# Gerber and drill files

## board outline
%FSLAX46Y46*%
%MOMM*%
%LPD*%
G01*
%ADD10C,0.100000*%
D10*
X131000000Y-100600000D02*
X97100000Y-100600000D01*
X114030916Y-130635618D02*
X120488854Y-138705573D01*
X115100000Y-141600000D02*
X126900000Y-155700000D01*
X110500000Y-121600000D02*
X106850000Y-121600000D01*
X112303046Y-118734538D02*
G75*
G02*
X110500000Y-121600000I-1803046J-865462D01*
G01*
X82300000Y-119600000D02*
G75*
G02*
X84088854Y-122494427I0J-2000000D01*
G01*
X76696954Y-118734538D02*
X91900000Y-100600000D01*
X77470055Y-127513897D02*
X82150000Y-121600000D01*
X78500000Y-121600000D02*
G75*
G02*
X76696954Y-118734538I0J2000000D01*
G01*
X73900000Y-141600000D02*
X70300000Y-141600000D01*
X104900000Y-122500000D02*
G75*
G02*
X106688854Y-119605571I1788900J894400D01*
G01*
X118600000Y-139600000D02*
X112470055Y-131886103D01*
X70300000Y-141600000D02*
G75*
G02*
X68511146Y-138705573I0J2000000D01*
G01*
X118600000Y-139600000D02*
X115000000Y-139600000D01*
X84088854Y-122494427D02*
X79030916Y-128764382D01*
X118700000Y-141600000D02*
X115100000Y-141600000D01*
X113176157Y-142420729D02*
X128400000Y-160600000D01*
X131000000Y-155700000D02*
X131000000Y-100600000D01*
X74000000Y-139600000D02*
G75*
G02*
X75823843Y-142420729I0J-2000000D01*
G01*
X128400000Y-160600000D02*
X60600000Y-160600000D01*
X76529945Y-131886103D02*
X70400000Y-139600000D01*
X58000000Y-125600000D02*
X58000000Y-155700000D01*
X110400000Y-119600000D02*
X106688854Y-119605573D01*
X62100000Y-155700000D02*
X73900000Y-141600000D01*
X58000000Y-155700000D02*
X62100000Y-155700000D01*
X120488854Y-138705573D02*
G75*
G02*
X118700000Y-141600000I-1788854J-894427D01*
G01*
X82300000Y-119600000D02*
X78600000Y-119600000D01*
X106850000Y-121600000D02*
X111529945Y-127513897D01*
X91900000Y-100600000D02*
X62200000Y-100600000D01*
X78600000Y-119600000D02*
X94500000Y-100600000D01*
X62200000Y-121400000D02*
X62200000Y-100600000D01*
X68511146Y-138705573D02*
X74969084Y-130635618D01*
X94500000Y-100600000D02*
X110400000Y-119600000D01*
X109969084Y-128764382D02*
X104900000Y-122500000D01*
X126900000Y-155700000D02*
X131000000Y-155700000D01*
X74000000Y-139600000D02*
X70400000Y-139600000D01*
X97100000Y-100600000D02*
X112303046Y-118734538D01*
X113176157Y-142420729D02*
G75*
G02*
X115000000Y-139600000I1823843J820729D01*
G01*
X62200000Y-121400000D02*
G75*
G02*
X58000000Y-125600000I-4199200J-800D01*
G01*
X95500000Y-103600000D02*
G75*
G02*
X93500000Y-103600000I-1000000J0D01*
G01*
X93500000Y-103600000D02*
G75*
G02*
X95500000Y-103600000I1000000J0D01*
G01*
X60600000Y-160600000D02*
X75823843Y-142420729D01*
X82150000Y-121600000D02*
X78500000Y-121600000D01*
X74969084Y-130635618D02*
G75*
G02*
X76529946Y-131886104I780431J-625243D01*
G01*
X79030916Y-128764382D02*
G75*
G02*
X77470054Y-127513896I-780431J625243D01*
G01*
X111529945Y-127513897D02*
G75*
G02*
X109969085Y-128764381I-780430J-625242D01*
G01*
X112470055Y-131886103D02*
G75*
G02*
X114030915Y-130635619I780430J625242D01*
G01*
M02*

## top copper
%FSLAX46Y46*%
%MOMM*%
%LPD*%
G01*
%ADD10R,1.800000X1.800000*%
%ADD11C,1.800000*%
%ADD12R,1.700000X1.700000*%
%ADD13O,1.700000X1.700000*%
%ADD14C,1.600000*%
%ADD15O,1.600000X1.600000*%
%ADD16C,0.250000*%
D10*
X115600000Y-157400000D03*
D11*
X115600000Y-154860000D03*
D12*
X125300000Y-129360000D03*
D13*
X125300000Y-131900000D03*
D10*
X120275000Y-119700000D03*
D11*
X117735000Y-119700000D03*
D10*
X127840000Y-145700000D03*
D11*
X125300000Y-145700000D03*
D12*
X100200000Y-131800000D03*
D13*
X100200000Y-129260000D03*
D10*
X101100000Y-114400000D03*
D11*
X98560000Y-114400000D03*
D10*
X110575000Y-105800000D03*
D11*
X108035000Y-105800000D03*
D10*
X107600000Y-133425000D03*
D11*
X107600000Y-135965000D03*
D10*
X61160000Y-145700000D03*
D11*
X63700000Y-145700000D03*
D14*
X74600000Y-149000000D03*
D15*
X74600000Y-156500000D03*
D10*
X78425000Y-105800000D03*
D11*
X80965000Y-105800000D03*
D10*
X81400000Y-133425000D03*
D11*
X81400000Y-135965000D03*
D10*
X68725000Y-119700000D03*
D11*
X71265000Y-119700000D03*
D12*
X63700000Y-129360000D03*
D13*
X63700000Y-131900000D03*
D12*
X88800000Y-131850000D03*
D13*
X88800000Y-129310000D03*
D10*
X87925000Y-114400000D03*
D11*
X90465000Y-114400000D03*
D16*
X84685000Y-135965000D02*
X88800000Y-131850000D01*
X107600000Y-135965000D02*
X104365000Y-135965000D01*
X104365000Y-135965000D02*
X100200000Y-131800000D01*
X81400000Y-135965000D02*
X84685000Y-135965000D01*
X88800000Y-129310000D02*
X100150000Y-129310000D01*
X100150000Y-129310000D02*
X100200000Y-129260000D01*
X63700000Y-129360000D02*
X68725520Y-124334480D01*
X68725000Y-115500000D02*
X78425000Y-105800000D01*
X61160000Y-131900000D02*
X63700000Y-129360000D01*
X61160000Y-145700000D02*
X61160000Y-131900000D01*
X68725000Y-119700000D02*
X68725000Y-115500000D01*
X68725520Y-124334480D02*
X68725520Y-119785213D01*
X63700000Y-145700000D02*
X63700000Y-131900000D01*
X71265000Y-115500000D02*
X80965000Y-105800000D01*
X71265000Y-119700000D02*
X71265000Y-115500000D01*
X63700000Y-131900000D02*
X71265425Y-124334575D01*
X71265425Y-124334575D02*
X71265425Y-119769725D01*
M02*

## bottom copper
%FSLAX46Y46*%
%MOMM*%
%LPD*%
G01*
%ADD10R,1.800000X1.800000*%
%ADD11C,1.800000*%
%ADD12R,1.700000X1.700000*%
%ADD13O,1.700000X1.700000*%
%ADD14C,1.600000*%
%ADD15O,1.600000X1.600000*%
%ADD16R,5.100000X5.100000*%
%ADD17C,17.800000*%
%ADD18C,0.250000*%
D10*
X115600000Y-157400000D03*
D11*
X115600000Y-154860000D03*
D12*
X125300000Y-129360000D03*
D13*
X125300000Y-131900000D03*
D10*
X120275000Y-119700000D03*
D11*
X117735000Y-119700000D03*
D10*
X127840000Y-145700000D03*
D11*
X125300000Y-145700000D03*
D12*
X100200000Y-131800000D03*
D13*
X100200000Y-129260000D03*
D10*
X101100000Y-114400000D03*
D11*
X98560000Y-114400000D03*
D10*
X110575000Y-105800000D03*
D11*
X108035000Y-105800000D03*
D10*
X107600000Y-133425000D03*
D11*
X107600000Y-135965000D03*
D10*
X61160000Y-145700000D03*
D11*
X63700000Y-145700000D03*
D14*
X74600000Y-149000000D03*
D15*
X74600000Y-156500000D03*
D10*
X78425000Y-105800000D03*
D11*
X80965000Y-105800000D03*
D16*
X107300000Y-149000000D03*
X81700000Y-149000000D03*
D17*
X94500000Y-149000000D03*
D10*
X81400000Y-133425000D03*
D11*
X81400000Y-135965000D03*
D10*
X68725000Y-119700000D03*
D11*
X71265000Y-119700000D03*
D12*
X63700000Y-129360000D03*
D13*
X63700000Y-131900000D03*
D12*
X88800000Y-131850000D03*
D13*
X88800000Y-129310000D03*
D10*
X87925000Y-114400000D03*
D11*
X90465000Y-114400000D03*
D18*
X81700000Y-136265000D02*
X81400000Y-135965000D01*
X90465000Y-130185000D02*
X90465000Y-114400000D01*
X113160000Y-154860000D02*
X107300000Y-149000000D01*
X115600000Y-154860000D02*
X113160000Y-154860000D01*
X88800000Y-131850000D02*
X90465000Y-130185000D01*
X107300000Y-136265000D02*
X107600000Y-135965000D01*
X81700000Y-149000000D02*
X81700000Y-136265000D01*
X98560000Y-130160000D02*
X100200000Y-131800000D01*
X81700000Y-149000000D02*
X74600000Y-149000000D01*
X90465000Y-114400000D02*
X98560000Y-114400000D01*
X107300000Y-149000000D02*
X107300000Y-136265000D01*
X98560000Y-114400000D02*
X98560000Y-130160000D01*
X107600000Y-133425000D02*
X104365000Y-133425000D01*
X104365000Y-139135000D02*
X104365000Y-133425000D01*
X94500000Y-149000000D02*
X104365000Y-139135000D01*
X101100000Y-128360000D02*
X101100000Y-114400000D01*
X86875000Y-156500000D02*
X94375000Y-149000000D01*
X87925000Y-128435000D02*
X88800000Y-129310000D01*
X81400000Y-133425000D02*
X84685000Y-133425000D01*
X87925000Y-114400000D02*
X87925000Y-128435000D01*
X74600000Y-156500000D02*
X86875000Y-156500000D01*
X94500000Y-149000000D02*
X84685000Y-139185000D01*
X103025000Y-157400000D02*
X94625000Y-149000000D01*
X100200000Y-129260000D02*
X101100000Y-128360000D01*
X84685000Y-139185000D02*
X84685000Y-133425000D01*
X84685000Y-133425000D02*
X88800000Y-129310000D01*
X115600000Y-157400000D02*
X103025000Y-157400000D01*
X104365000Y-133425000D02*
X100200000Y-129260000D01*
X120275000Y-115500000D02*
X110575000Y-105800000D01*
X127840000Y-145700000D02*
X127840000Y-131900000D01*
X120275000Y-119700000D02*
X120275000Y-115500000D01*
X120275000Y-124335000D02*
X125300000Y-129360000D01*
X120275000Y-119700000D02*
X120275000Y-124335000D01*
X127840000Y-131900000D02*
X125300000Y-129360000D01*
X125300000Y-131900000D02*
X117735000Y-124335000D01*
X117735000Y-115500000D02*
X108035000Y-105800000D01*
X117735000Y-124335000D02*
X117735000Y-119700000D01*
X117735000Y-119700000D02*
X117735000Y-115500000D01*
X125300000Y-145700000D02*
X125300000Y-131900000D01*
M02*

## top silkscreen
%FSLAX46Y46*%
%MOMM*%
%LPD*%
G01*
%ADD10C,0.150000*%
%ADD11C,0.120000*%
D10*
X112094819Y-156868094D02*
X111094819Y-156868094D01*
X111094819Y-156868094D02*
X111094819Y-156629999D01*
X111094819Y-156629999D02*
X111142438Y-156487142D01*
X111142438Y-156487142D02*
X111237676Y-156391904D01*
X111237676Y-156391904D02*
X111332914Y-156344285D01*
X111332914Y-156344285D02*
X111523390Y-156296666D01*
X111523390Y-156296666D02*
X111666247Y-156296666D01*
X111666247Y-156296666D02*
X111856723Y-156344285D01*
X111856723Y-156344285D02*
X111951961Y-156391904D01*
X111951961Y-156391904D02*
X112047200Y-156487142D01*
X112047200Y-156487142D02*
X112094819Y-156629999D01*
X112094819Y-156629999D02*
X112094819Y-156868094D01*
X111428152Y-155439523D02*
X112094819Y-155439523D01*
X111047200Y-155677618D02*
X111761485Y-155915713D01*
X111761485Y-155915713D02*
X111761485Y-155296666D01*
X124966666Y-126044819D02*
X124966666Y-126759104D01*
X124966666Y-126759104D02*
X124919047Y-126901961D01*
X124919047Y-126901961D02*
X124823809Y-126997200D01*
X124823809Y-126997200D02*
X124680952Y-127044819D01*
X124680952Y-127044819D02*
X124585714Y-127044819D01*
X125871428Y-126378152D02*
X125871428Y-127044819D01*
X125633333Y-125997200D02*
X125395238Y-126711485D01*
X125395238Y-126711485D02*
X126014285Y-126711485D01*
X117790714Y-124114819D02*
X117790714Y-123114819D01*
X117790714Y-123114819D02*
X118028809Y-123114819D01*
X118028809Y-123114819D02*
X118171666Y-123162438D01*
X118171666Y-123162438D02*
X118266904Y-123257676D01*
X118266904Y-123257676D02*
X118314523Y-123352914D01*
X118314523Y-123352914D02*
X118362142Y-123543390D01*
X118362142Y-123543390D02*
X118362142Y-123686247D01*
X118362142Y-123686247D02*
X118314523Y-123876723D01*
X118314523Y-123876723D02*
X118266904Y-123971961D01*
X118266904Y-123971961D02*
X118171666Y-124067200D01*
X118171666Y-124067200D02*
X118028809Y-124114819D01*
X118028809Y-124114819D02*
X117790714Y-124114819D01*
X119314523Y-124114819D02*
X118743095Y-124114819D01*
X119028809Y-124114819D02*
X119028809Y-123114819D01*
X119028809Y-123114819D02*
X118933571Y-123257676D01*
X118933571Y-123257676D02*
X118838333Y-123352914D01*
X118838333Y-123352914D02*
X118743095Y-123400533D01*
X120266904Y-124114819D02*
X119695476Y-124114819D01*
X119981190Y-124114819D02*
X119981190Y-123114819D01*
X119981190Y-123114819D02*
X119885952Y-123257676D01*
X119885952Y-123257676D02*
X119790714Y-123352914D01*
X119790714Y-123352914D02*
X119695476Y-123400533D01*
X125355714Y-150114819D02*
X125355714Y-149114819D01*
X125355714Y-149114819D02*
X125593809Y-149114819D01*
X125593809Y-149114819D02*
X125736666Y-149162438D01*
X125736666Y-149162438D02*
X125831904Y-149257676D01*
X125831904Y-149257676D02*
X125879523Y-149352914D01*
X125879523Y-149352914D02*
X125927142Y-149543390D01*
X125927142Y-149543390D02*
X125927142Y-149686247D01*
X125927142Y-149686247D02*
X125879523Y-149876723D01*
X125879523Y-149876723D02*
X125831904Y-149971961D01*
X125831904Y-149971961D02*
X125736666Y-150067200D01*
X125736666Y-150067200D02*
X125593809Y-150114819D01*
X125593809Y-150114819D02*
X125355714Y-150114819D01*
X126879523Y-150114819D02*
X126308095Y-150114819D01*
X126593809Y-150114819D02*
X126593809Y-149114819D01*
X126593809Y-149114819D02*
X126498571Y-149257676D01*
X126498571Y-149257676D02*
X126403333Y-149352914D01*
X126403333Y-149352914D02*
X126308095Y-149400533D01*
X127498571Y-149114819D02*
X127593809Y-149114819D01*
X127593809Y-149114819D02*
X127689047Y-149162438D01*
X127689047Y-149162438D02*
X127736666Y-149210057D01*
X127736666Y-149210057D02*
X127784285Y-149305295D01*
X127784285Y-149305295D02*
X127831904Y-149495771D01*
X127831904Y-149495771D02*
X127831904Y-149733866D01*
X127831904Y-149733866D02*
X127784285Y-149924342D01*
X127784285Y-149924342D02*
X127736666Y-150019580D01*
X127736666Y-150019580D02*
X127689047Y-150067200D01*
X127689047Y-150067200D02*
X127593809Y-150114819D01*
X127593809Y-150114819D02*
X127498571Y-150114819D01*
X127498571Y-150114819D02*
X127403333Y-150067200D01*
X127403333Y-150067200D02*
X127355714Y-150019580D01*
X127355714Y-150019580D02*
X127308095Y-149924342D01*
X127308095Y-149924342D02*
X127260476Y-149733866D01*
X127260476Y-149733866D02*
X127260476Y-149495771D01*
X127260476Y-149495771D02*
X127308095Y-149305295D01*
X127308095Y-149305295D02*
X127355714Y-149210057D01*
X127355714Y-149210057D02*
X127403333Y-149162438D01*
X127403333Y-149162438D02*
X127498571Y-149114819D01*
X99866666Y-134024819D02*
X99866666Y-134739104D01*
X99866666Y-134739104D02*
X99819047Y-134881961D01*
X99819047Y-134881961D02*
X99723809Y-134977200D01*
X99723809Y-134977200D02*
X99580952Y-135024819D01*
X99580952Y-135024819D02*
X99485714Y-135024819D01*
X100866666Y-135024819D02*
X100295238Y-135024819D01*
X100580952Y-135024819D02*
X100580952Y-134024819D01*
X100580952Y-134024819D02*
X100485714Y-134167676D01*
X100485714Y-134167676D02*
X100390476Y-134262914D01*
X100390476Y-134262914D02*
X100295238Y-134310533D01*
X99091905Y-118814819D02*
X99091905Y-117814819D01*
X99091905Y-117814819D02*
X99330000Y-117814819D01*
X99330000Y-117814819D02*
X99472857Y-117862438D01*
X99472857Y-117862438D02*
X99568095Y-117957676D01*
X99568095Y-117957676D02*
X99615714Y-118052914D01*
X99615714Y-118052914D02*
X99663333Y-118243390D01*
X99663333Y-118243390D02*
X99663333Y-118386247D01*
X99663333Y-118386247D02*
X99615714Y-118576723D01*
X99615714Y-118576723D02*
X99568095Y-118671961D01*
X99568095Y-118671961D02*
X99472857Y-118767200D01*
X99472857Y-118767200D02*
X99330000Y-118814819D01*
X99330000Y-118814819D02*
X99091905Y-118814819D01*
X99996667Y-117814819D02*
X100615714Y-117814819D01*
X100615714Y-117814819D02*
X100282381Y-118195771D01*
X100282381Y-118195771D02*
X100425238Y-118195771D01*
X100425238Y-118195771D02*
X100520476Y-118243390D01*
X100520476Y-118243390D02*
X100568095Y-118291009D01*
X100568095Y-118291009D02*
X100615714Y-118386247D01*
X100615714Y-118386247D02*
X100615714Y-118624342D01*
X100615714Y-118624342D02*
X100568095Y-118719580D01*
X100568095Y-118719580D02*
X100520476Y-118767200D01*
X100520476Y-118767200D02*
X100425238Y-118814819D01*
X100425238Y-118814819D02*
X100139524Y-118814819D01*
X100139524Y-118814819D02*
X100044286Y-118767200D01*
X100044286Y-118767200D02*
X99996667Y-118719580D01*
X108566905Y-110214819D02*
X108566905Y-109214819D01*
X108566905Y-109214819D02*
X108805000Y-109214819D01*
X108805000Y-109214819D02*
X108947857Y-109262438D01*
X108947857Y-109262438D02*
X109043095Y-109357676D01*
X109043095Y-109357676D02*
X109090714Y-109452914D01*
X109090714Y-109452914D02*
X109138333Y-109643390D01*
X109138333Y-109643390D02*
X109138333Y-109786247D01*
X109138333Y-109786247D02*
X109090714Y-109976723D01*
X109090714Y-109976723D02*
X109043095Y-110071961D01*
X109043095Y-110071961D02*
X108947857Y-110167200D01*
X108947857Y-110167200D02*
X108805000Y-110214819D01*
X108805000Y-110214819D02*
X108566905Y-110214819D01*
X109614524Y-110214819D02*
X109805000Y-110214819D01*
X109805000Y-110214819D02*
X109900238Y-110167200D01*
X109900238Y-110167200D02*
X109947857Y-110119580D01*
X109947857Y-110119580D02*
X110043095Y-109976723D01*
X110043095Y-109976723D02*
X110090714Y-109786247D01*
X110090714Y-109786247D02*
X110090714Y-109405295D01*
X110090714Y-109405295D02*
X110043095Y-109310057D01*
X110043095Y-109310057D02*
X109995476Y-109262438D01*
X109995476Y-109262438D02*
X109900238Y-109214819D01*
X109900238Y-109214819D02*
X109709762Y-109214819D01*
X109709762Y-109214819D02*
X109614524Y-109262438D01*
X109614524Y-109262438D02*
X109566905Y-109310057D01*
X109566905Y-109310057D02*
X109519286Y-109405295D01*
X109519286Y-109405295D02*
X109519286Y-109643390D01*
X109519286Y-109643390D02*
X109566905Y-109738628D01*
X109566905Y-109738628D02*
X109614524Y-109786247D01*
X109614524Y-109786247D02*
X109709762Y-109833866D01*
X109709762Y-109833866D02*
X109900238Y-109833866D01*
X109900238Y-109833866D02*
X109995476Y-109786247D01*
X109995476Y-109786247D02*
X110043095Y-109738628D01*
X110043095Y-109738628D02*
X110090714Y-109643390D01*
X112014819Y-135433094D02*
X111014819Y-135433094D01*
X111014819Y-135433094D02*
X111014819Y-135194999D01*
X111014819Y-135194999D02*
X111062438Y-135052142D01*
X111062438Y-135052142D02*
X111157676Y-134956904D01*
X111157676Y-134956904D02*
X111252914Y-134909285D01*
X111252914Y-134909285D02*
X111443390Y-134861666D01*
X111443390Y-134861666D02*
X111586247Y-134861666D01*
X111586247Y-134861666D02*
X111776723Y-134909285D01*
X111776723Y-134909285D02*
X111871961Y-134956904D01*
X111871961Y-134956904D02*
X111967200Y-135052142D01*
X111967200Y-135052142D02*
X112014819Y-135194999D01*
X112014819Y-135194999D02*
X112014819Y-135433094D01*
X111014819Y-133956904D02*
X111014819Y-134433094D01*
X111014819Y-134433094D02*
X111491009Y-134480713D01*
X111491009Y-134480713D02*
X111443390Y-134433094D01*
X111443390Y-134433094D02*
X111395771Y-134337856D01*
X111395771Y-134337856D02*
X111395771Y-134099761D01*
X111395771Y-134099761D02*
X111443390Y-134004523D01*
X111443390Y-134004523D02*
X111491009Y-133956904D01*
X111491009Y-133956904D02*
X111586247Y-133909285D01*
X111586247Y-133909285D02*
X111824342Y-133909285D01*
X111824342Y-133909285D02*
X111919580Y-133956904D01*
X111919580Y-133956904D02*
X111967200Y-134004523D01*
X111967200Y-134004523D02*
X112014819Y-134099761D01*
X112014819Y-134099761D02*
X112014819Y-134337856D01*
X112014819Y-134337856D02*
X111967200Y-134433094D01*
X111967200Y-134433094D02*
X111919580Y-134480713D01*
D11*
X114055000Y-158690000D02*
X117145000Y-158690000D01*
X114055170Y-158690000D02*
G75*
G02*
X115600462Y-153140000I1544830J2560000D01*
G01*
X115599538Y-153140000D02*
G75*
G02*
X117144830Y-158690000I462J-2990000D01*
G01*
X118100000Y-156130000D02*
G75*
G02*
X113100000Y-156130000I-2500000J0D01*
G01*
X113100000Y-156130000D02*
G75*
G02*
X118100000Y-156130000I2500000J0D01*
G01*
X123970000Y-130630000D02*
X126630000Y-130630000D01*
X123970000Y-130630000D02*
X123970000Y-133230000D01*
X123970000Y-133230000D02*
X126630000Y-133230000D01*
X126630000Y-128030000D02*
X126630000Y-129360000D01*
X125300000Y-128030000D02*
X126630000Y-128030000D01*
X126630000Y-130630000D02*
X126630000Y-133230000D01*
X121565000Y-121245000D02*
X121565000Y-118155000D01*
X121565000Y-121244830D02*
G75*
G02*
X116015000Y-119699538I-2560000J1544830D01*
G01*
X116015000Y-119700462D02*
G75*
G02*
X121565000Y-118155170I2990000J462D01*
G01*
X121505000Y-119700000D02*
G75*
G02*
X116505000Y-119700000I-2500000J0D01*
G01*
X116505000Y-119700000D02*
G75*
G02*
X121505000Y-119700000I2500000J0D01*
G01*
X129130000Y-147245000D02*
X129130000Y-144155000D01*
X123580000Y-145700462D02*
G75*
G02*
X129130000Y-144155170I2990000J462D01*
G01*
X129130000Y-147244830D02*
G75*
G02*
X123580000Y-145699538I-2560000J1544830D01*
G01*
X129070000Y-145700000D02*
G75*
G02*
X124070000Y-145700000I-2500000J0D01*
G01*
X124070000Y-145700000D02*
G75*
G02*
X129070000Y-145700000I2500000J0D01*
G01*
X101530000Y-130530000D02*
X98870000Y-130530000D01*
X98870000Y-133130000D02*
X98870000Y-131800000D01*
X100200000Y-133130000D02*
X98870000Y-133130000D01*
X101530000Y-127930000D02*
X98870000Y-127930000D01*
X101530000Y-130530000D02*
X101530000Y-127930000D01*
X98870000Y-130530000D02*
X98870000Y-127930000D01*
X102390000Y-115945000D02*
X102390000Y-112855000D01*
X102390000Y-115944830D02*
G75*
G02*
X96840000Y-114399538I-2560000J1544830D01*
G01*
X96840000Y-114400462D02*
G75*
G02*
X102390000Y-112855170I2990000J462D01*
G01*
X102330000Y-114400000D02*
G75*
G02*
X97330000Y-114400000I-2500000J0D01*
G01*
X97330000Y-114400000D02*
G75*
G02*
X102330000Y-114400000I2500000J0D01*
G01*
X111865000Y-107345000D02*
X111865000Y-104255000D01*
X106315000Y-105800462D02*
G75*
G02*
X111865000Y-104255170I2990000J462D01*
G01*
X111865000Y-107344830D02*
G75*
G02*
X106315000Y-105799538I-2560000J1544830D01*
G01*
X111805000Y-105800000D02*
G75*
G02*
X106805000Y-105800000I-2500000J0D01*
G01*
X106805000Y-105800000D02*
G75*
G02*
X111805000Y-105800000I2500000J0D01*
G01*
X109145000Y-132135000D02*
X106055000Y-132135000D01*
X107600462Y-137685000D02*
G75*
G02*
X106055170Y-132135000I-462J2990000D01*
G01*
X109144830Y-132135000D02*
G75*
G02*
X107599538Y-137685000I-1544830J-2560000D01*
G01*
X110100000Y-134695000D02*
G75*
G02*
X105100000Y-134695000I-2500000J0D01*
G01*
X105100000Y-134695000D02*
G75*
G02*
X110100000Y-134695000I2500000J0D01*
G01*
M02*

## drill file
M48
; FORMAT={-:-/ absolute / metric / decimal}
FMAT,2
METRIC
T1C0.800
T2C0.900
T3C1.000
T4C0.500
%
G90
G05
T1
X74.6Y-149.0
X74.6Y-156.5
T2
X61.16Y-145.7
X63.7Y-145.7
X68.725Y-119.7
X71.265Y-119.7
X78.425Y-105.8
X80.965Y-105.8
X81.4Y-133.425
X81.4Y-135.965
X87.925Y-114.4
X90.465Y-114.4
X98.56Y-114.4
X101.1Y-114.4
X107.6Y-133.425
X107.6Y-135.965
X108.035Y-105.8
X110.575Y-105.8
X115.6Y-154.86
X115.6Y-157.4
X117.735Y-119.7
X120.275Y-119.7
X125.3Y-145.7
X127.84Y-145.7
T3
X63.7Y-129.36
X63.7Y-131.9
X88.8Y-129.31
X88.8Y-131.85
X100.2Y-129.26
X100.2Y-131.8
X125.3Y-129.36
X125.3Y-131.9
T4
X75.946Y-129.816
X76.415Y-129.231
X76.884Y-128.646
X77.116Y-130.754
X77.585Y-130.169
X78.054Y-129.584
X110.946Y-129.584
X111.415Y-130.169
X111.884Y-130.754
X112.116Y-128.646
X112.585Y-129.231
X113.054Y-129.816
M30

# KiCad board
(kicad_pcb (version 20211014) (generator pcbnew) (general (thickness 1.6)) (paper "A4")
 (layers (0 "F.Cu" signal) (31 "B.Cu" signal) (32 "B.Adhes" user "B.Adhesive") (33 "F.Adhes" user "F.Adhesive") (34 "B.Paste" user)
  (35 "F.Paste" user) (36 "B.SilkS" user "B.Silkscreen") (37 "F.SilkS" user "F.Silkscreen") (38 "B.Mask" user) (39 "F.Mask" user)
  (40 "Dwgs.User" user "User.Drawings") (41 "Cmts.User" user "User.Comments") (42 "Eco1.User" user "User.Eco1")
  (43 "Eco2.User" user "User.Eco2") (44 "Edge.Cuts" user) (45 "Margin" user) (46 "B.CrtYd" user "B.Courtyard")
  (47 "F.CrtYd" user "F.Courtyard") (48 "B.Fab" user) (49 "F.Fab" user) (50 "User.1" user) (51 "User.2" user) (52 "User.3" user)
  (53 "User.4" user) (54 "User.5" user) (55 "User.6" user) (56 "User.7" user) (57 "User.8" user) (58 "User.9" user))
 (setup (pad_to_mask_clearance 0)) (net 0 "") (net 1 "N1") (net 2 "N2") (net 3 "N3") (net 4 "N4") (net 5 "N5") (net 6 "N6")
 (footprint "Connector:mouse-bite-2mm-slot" (layer "F.Cu") (at 77 129.7 -128.7)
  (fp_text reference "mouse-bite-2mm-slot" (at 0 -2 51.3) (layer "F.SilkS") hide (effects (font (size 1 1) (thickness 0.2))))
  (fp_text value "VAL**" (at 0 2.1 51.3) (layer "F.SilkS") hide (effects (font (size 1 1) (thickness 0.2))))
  (fp_arc (start 2 1) (mid 1 0) (end 2 -1) (layer "Edge.Cuts") (width 0.1))
  (fp_arc (start -2 -1) (mid -1 0) (end -2 1) (layer "Edge.Cuts") (width 0.1))
  (pad "" np_thru_hole circle (at 0.75 0.75 231.3) (size 0.5 0.5) (drill 0.5) (layers F&B.Cu *.Mask))
  (pad "" np_thru_hole circle (at 0.75 -0.75 231.3) (size 0.5 0.5) (drill 0.5) (layers F&B.Cu *.Mask))
  (pad "" np_thru_hole circle (at 0 0.75 231.3) (size 0.5 0.5) (drill 0.5) (layers F&B.Cu *.Mask))
  (pad "" np_thru_hole circle (at 0 -0.75 231.3) (size 0.5 0.5) (drill 0.5) (layers F&B.Cu *.Mask))
  (pad "" np_thru_hole circle (at -0.75 0.75 231.3) (size 0.5 0.5) (drill 0.5) (layers F&B.Cu *.Mask))
  (pad "" np_thru_hole circle (at -0.75 -0.75 231.3) (size 0.5 0.5) (drill 0.5) (layers F&B.Cu *.Mask)))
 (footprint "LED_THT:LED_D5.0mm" (layer "F.Cu") (at 115.6 157.4 90)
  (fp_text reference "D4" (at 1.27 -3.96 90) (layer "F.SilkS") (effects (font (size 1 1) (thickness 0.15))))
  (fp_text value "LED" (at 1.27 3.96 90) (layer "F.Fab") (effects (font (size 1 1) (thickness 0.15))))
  (fp_line (start -1.29 -1.545) (end -1.29 1.545) (layer "F.SilkS") (width 0.12))
  (fp_arc (start -1.29 -1.54483) (mid 2.072002 -2.880433) (end 4.26 0.000462) (layer "F.SilkS") (width 0.12))
  (fp_arc (start 4.26 -0.000462) (mid 2.072002 2.880433) (end -1.29 1.54483) (layer "F.SilkS") (width 0.12))
  (fp_circle (center 1.27 0) (end 3.77 0) (layer "F.SilkS") (width 0.12) (fill none))
  (pad "1" thru_hole rect (at 0 0 90) (size 1.8 1.8) (drill 0.9) (layers *.Cu *.Mask) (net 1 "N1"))
  (pad "2" thru_hole circle (at 2.54 0 90) (size 1.8 1.8) (drill 0.9) (layers *.Cu *.Mask) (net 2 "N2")))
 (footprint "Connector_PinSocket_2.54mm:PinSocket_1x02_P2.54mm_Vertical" (layer "F.Cu") (at 125.3 129.36)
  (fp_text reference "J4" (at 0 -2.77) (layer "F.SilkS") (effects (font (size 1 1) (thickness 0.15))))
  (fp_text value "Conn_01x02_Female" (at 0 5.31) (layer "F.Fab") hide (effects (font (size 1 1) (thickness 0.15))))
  (fp_line (start -1.33 1.27) (end 1.33 1.27) (layer "F.SilkS") (width 0.12))
  (fp_line (start -1.33 1.27) (end -1.33 3.87) (layer "F.SilkS") (width 0.12))
  (fp_line (start -1.33 3.87) (end 1.33 3.87) (layer "F.SilkS") (width 0.12))
  (fp_line (start 1.33 -1.33) (end 1.33 0) (layer "F.SilkS") (width 0.12))
  (fp_line (start 0 -1.33) (end 1.33 -1.33) (layer "F.SilkS") (width 0.12))
  (fp_line (start 1.33 1.27) (end 1.33 3.87) (layer "F.SilkS") (width 0.12))
  (pad "1" thru_hole rect (at 0 0) (size 1.7 1.7) (drill 1) (layers *.Cu *.Mask) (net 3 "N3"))
  (pad "2" thru_hole oval (at 0 2.54) (size 1.7 1.7) (drill 1) (layers *.Cu *.Mask) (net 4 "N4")))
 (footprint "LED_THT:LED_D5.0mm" (layer "F.Cu") (at 120.275 119.7 180)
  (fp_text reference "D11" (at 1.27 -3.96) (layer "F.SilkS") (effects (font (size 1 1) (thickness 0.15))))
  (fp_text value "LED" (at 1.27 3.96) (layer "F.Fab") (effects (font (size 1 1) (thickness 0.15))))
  (fp_line (start -1.29 -1.545) (end -1.29 1.545) (layer "F.SilkS") (width 0.12))
  (fp_arc (start -1.29 -1.54483) (mid 2.072002 -2.880433) (end 4.26 0.000462) (layer "F.SilkS") (width 0.12))
  (fp_arc (start 4.26 -0.000462) (mid 2.072002 2.880433) (end -1.29 1.54483) (layer "F.SilkS") (width 0.12))
  (fp_circle (center 1.27 0) (end 3.77 0) (layer "F.SilkS") (width 0.12) (fill none))
  (pad "1" thru_hole rect (at 0 0 180) (size 1.8 1.8) (drill 0.9) (layers *.Cu *.Mask) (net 3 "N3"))
  (pad "2" thru_hole circle (at 2.54 0 180) (size 1.8 1.8) (drill 0.9) (layers *.Cu *.Mask) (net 4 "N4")))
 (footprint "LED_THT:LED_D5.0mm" (layer "F.Cu") (at 127.84 145.7 180)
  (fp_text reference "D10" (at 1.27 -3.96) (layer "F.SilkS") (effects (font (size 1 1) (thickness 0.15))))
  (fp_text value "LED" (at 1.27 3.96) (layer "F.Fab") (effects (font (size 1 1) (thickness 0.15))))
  (fp_line (start -1.29 -1.545) (end -1.29 1.545) (layer "F.SilkS") (width 0.12))
  (fp_arc (start 4.26 -0.000462) (mid 2.072002 2.880433) (end -1.29 1.54483) (layer "F.SilkS") (width 0.12))
  (fp_arc (start -1.29 -1.54483) (mid 2.072002 -2.880433) (end 4.26 0.000462) (layer "F.SilkS") (width 0.12))
  (fp_circle (center 1.27 0) (end 3.77 0) (layer "F.SilkS") (width 0.12) (fill none))
  (pad "1" thru_hole rect (at 0 0 180) (size 1.8 1.8) (drill 0.9) (layers *.Cu *.Mask) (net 3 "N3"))
  (pad "2" thru_hole circle (at 2.54 0 180) (size 1.8 1.8) (drill 0.9) (layers *.Cu *.Mask) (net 4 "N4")))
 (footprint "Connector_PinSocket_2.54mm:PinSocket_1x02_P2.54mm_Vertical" (layer "F.Cu") (at 100.2 131.8 180)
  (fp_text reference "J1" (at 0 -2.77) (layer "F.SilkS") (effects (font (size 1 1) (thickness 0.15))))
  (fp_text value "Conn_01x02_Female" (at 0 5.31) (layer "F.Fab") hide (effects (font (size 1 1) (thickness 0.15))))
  (fp_line (start -1.33 1.27) (end 1.33 1.27) (layer "F.SilkS") (width 0.12))
  (fp_line (start 1.33 -1.33) (end 1.33 0) (layer "F.SilkS") (width 0.12))
  (fp_line (start 0 -1.33) (end 1.33 -1.33) (layer "F.SilkS") (width 0.12))
  (fp_line (start -1.33 3.87) (end 1.33 3.87) (layer "F.SilkS") (width 0.12))
  (fp_line (start -1.33 1.27) (end -1.33 3.87) (layer "F.SilkS") (width 0.12))
  (fp_line (start 1.33 1.27) (end 1.33 3.87) (layer "F.SilkS") (width 0.12))
  (pad "1" thru_hole rect (at 0 0 180) (size 1.7 1.7) (drill 1) (layers *.Cu *.Mask) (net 2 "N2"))
  (pad "2" thru_hole oval (at 0 2.54 180) (size 1.7 1.7) (drill 1) (layers *.Cu *.Mask) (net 1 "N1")))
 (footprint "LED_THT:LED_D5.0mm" (layer "F.Cu") (at 101.1 114.4 180)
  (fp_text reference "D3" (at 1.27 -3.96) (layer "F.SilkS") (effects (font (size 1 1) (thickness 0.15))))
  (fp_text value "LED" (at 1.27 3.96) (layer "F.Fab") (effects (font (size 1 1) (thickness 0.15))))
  (fp_line (start -1.29 -1.545) (end -1.29 1.545) (layer "F.SilkS") (width 0.12))
  (fp_arc (start -1.29 -1.54483) (mid 2.072002 -2.880433) (end 4.26 0.000462) (layer "F.SilkS") (width 0.12))
  (fp_arc (start 4.26 -0.000462) (mid 2.072002 2.880433) (end -1.29 1.54483) (layer "F.SilkS") (width 0.12))
  (fp_circle (center 1.27 0) (end 3.77 0) (layer "F.SilkS") (width 0.12) (fill none))
  (pad "1" thru_hole rect (at 0 0 180) (size 1.8 1.8) (drill 0.9) (layers *.Cu *.Mask) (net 1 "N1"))
  (pad "2" thru_hole circle (at 2.54 0 180) (size 1.8 1.8) (drill 0.9) (layers *.Cu *.Mask) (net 2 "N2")))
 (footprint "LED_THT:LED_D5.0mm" (layer "F.Cu") (at 110.575 105.8 180)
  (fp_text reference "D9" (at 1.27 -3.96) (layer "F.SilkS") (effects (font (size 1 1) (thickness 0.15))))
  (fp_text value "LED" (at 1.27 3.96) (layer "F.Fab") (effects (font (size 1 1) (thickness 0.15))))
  (fp_line (start -1.29 -1.545) (end -1.29 1.545) (layer "F.SilkS") (width 0.12))
  (fp_arc (start 4.26 -0.000462) (mid 2.072002 2.880433) (end -1.29 1.54483) (layer "F.SilkS") (width 0.12))
  (fp_arc (start -1.29 -1.54483) (mid 2.072002 -2.880433) (end 4.26 0.000462) (layer "F.SilkS") (width 0.12))
  (fp_circle (center 1.27 0) (end 3.77 0) (layer "F.SilkS") (width 0.12) (fill none))
  (pad "1" thru_hole rect (at 0 0 180) (size 1.8 1.8) (drill 0.9) (layers *.Cu *.Mask) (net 3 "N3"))
  (pad "2" thru_hole circle (at 2.54 0 180) (size 1.8 1.8) (drill 0.9) (layers *.Cu *.Mask) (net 4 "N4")))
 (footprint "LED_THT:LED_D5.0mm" (layer "F.Cu") (at 107.6 133.425 -90)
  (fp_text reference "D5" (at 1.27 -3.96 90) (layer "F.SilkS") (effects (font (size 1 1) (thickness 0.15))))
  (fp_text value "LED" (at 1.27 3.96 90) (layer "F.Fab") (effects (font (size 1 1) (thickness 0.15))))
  (fp_line (start -1.29 -1.545) (end -1.29 1.545) (layer "F.SilkS") (width 0.12))
  (fp_arc (start 4.26 -0.000462) (mid 2.072002 2.880433) (end -1.29 1.54483) (layer "F.SilkS") (width 0.12))
  (fp_arc (start -1.29 -1.54483) (mid 2.072002 -2.880433) (end 4.26 0.000462) (layer "F.SilkS") (width 0.12))
  (fp_circle (center 1.27 0) (end 3.77 0) (layer "F.SilkS") (width 0.12) (fill none))
  (pad "1" thru_hole rect (at 0 0 270) (size 1.8 1.8) (drill 0.9) (layers *.Cu *.Mask) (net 1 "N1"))
  (pad "2" thru_hole circle (at 2.54 0 270) (size 1.8 1.8) (drill 0.9) (layers *.Cu *.Mask) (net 2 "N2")))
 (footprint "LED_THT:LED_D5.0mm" (layer "B.Cu") (at 61.16 145.7)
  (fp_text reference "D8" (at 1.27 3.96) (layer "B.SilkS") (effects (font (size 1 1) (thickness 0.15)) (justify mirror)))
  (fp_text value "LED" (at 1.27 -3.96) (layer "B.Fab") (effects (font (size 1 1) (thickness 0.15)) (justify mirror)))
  (pad "1" thru_hole rect (at 0 0) (size 1.8 1.8) (drill 0.9) (layers *.Cu *.Mask) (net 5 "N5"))
  (pad "2" thru_hole circle (at 2.54 0) (size 1.8 1.8) (drill 0.9) (layers *.Cu *.Mask) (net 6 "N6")))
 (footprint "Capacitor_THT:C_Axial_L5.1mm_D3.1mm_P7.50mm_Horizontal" (layer "B.Cu") (at 74.6 149 -90)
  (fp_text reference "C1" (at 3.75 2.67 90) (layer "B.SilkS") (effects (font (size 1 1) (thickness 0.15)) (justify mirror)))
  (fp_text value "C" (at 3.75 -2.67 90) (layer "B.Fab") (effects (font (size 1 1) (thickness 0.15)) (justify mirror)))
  (pad "1" thru_hole circle (at 0 0 270) (size 1.6 1.6) (drill 0.8) (layers *.Cu *.Mask) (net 2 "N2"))
  (pad "2" thru_hole oval (at 7.5 0 270) (size 1.6 1.6) (drill 0.8) (layers *.Cu *.Mask) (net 1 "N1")))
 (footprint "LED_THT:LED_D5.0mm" (layer "B.Cu") (at 78.425 105.8)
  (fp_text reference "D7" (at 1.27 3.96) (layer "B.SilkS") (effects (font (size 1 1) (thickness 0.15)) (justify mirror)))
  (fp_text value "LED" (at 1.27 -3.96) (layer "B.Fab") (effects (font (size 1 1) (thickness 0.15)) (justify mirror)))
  (pad "1" thru_hole rect (at 0 0) (size 1.8 1.8) (drill 0.9) (layers *.Cu *.Mask) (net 5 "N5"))
  (pad "2" thru_hole circle (at 2.54 0) (size 1.8 1.8) (drill 0.9) (layers *.Cu *.Mask) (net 6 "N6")))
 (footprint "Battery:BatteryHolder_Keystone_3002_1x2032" (layer "B.Cu") (at 94.5 149)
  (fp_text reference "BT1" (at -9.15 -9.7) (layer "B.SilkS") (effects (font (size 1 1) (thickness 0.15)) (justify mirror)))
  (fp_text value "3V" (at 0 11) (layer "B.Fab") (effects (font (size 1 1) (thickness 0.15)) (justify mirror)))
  (pad "1" smd rect (at 12.8 0) (size 5.1 5.1) (layers "B.Cu" "B.Paste" "B.Mask") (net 2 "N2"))
  (pad "1" smd rect (at -12.8 0) (size 5.1 5.1) (layers "B.Cu" "B.Paste" "B.Mask") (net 2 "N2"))
  (pad "2" smd circle (at 0 0) (size 17.8 17.8) (layers "B.Cu" "B.Mask") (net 1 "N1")))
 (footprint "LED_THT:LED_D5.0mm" (layer "B.Cu") (at 81.4 133.425 -90)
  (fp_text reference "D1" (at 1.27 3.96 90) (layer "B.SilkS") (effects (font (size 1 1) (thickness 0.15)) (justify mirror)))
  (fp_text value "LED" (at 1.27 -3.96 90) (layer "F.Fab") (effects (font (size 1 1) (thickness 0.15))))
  (pad "1" thru_hole rect (at 0 0 270) (size 1.8 1.8) (drill 0.9) (layers *.Cu *.Mask) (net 1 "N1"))
  (pad "2" thru_hole circle (at 2.54 0 270) (size 1.8 1.8) (drill 0.9) (layers *.Cu *.Mask) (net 2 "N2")))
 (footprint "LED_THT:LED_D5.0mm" (layer "B.Cu") (at 68.725 119.7)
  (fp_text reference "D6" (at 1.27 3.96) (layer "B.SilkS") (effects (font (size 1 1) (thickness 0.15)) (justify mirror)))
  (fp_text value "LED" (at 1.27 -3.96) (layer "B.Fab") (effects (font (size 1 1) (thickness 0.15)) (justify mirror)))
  (pad "1" thru_hole rect (at 0 0) (size 1.8 1.8) (drill 0.9) (layers *.Cu *.Mask) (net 5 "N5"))
  (pad "2" thru_hole circle (at 2.54 0) (size 1.8 1.8) (drill 0.9) (layers *.Cu *.Mask) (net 6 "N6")))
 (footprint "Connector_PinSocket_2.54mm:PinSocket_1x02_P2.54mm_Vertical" (layer "B.Cu") (at 63.7 129.36 180)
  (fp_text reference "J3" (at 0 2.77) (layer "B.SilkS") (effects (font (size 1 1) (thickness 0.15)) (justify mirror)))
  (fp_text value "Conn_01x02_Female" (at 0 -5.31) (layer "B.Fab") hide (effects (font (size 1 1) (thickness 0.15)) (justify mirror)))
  (pad "1" thru_hole rect (at 0 0 180) (size 1.7 1.7) (drill 1) (layers *.Cu *.Mask) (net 5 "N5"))
  (pad "2" thru_hole oval (at 0 -2.54 180) (size 1.7 1.7) (drill 1) (layers *.Cu *.Mask) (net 6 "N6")))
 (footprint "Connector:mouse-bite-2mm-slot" (layer "B.Cu") (at 112 129.7 -51.3)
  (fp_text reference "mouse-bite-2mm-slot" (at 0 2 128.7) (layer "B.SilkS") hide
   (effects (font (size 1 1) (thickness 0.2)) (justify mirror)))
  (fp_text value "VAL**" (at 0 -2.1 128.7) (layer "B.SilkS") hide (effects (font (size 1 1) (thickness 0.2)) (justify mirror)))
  (fp_arc (start -2 -1) (mid -1 0) (end -2 1) (layer "Edge.Cuts") (width 0.1))
  (fp_arc (start 2 1) (mid 1 0) (end 2 -1) (layer "Edge.Cuts") (width 0.1))
  (pad "" np_thru_hole circle (at 0.75 -0.75 308.7) (size 0.5 0.5) (drill 0.5) (layers *.Cu *.Mask))
  (pad "" np_thru_hole circle (at 0 0.75 308.7) (size 0.5 0.5) (drill 0.5) (layers *.Cu *.Mask))
  (pad "" np_thru_hole circle (at -0.75 0.75 308.7) (size 0.5 0.5) (drill 0.5) (layers *.Cu *.Mask))
  (pad "" np_thru_hole circle (at 0 -0.75 308.7) (size 0.5 0.5) (drill 0.5) (layers *.Cu *.Mask))
  (pad "" np_thru_hole circle (at 0.75 0.75 308.7) (size 0.5 0.5) (drill 0.5) (layers *.Cu *.Mask))
  (pad "" np_thru_hole circle (at -0.75 -0.75 308.7) (size 0.5 0.5) (drill 0.5) (layers *.Cu *.Mask)))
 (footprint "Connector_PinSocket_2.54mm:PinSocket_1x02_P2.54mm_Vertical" (layer "B.Cu") (at 88.8 131.85)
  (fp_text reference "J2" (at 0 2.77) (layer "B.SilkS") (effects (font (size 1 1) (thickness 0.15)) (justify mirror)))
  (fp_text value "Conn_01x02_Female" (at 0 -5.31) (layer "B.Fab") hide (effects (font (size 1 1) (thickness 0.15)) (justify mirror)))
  (pad "1" thru_hole rect (at 0 0) (size 1.7 1.7) (drill 1) (layers *.Cu *.Mask) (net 2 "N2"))
  (pad "2" thru_hole oval (at 0 -2.54) (size 1.7 1.7) (drill 1) (layers *.Cu *.Mask) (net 1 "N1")))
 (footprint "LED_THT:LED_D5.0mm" (layer "B.Cu") (at 87.925 114.4)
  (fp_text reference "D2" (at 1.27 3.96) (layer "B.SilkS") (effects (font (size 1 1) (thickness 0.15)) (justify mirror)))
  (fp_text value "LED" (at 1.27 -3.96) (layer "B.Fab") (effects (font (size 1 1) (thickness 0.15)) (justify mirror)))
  (pad "1" thru_hole rect (at 0 0) (size 1.8 1.8) (drill 0.9) (layers *.Cu *.Mask) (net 1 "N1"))
  (pad "2" thru_hole circle (at 2.54 0) (size 1.8 1.8) (drill 0.9) (layers *.Cu *.Mask) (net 2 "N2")))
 (gr_line (start 131 100.6) (end 97.1 100.6) (layer "Edge.Cuts") (width 0.1))
 (gr_line (start 114.030916 130.635618) (end 120.488854 138.705573) (layer "Edge.Cuts") (width 0.1))
 (gr_line (start 115.1 141.6) (end 126.9 155.7) (layer "Edge.Cuts") (width 0.1))
 (gr_line (start 110.5 121.6) (end 106.85 121.6) (layer "Edge.Cuts") (width 0.1))
 (gr_arc (start 112.303046 118.734538) (mid 112.192767 120.665147) (end 110.5 121.6) (layer "Edge.Cuts") (width 0.1))
 (gr_arc (start 82.3 119.6) (mid 84.001302 120.548538) (end 84.088854 122.494427) (layer "Edge.Cuts") (width 0.1))
 (gr_line (start 76.696954 118.734538) (end 91.9 100.6) (layer "Edge.Cuts") (width 0.1))
 (gr_line (start 77.470055 127.513897) (end 82.15 121.6) (layer "Edge.Cuts") (width 0.1))
 (gr_arc (start 78.5 121.6) (mid 76.807232 120.665147) (end 76.696954 118.734538) (layer "Edge.Cuts") (width 0.1))
 (gr_line (start 73.9 141.6) (end 70.3 141.6) (layer "Edge.Cuts") (width 0.1))
 (gr_arc (start 104.9 122.5) (mid 104.987574 120.554123) (end 106.688854 119.605573) (layer "Edge.Cuts") (width 0.1))
 (gr_line (start 118.6 139.6) (end 112.470055 131.886103) (layer "Edge.Cuts") (width 0.1))
 (gr_arc (start 70.3 141.6) (mid 68.598698 140.651462) (end 68.511146 138.705573) (layer "Edge.Cuts") (width 0.1))
 (gr_line (start 118.6 139.6) (end 115 139.6) (layer "Edge.Cuts") (width 0.1))
 (gr_line (start 84.088854 122.494427) (end 79.030916 128.764382) (layer "Edge.Cuts") (width 0.1))
 (gr_line (start 118.7 141.6) (end 115.1 141.6) (layer "Edge.Cuts") (width 0.1))
 (gr_line (start 113.176157 142.420729) (end 128.4 160.6) (layer "Edge.Cuts") (width 0.1))
 (gr_line (start 131 155.7) (end 131 100.6) (layer "Edge.Cuts") (width 0.1))
 (gr_arc (start 74 139.6) (mid 75.679503 140.514058) (end 75.823843 142.420729) (layer "Edge.Cuts") (width 0.1))
 (gr_line (start 128.4 160.6) (end 60.6 160.6) (layer "Edge.Cuts") (width 0.1))
 (gr_line (start 76.529945 131.886103) (end 70.4 139.6) (layer "Edge.Cuts") (width 0.1))
 (gr_line (start 58 125.6) (end 58 155.7) (layer "Edge.Cuts") (width 0.1))
 (gr_line (start 110.4 119.6) (end 106.688854 119.605573) (layer "Edge.Cuts") (width 0.1))
 (gr_line (start 62.1 155.7) (end 73.9 141.6) (layer "Edge.Cuts") (width 0.1))
 (gr_line (start 58 155.7) (end 62.1 155.7) (layer "Edge.Cuts") (width 0.1))
 (gr_arc (start 120.488854 138.705573) (mid 120.401301 140.651462) (end 118.7 141.6) (layer "Edge.Cuts") (width 0.1))
 (gr_line (start 82.3 119.6) (end 78.6 119.6) (layer "Edge.Cuts") (width 0.1))
 (gr_line (start 106.85 121.6) (end 111.529945 127.513897) (layer "Edge.Cuts") (width 0.1))
 (gr_line (start 91.9 100.6) (end 62.2 100.6) (layer "Edge.Cuts") (width 0.1))
 (gr_line (start 78.6 119.6) (end 94.5 100.6) (layer "Edge.Cuts") (width 0.1))
 (gr_line (start 62.2 121.4) (end 62.2 100.6) (layer "Edge.Cuts") (width 0.1))
 (gr_line (start 68.511146 138.705573) (end 74.969084 130.635618) (layer "Edge.Cuts") (width 0.1))
 (gr_line (start 94.5 100.6) (end 110.4 119.6) (layer "Edge.Cuts") (width 0.1))
 (gr_line (start 109.969084 128.764382) (end 104.9 122.5) (layer "Edge.Cuts") (width 0.1))
 (gr_line (start 126.9 155.7) (end 131 155.7) (layer "Edge.Cuts") (width 0.1))
 (gr_line (start 74 139.6) (end 70.4 139.6) (layer "Edge.Cuts") (width 0.1))
 (gr_line (start 97.1 100.6) (end 112.303046 118.734538) (layer "Edge.Cuts") (width 0.1))
 (gr_arc (start 113.176157 142.420729) (mid 113.320498 140.514058) (end 115 139.6) (layer "Edge.Cuts") (width 0.1))
 (gr_arc (start 62.2 121.4) (mid 60.970083 124.370083) (end 58 125.6) (layer "Edge.Cuts") (width 0.1))
 (gr_circle (center 94.5 103.6) (end 94.5 104.6) (layer "Edge.Cuts") (width 0.1) (fill none))
 (gr_line (start 60.6 160.6) (end 75.823843 142.420729) (layer "Edge.Cuts") (width 0.1))
 (gr_line (start 82.15 121.6) (end 78.5 121.6) (layer "Edge.Cuts") (width 0.1))
 (segment (start 84.685 135.965) (end 88.8 131.85) (width 0.25) (layer "F.Cu") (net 2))
 (segment (start 107.6 135.965) (end 104.365 135.965) (width 0.25) (layer "F.Cu") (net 2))
 (segment (start 104.365 135.965) (end 100.2 131.8) (width 0.25) (layer "F.Cu") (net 2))
 (segment (start 81.4 135.965) (end 84.685 135.965) (width 0.25) (layer "F.Cu") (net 2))
 (segment (start 81.7 136.265) (end 81.4 135.965) (width 0.25) (layer "B.Cu") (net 2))
 (segment (start 90.465 130.185) (end 90.465 114.4) (width 0.25) (layer "B.Cu") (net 2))
 (segment (start 113.16 154.86) (end 107.3 149) (width 0.25) (layer "B.Cu") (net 2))
 (segment (start 115.6 154.86) (end 113.16 154.86) (width 0.25) (layer "B.Cu") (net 2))
 (segment (start 88.8 131.85) (end 90.465 130.185) (width 0.25) (layer "B.Cu") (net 2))
 (segment (start 107.3 136.265) (end 107.6 135.965) (width 0.25) (layer "B.Cu") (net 2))
 (segment (start 81.7 149) (end 81.7 136.265) (width 0.25) (layer "B.Cu") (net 2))
 (segment (start 98.56 130.16) (end 100.2 131.8) (width 0.25) (layer "B.Cu") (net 2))
 (segment (start 81.7 149) (end 74.6 149) (width 0.25) (layer "B.Cu") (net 2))
 (segment (start 90.465 114.4) (end 98.56 114.4) (width 0.25) (layer "B.Cu") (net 2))
 (segment (start 107.3 149) (end 107.3 136.265) (width 0.25) (layer "B.Cu") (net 2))
 (segment (start 98.56 114.4) (end 98.56 130.16) (width 0.25) (layer "B.Cu") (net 2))
 (segment (start 88.8 129.31) (end 100.15 129.31) (width 0.25) (layer "F.Cu") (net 1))
 (segment (start 100.15 129.31) (end 100.2 129.26) (width 0.25) (layer "F.Cu") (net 1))
 (segment (start 107.6 133.425) (end 104.365 133.425) (width 0.25) (layer "B.Cu") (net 1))
 (segment (start 104.365 139.135) (end 104.365 133.425) (width 0.25) (layer "B.Cu") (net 1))
 (segment (start 94.5 149) (end 104.365 139.135) (width 0.25) (layer "B.Cu") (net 1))
 (segment (start 101.1 128.36) (end 101.1 114.4) (width 0.25) (layer "B.Cu") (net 1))
 (segment (start 86.875 156.5) (end 94.375 149) (width 0.25) (layer "B.Cu") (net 1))
 (segment (start 87.925 128.435) (end 88.8 129.31) (width 0.25) (layer "B.Cu") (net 1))
 (segment (start 81.4 133.425) (end 84.685 133.425) (width 0.25) (layer "B.Cu") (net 1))
 (segment (start 87.925 114.4) (end 87.925 128.435) (width 0.25) (layer "B.Cu") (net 1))
 (segment (start 74.6 156.5) (end 86.875 156.5) (width 0.25) (layer "B.Cu") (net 1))
 (segment (start 94.5 149) (end 84.685 139.185) (width 0.25) (layer "B.Cu") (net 1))
 (segment (start 103.025 157.4) (end 94.625 149) (width 0.25) (layer "B.Cu") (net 1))
 (segment (start 100.2 129.26) (end 101.1 128.36) (width 0.25) (layer "B.Cu") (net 1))
 (segment (start 84.685 139.185) (end 84.685 133.425) (width 0.25) (layer "B.Cu") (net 1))
 (segment (start 84.685 133.425) (end 88.8 129.31) (width 0.25) (layer "B.Cu") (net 1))
 (segment (start 115.6 157.4) (end 103.025 157.4) (width 0.25) (layer "B.Cu") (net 1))
 (segment (start 104.365 133.425) (end 100.2 129.26) (width 0.25) (layer "B.Cu") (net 1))
 (segment (start 63.7 129.36) (end 68.72552 124.33448) (width 0.25) (layer "F.Cu") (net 5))
 (segment (start 68.725 115.5) (end 78.425 105.8) (width 0.25) (layer "F.Cu") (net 5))
 (segment (start 61.16 131.9) (end 63.7 129.36) (width 0.25) (layer "F.Cu") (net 5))
 (segment (start 61.16 145.7) (end 61.16 131.9) (width 0.25) (layer "F.Cu") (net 5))
 (segment (start 68.725 119.7) (end 68.725 115.5) (width 0.25) (layer "F.Cu") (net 5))
 (segment (start 68.72552 124.33448) (end 68.72552 119.785213) (width 0.25) (layer "F.Cu") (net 5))
 (segment (start 63.7 145.7) (end 63.7 131.9) (width 0.25) (layer "F.Cu") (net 6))
 (segment (start 71.265 115.5) (end 80.965 105.8) (width 0.25) (layer "F.Cu") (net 6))
 (segment (start 71.265 119.7) (end 71.265 115.5) (width 0.25) (layer "F.Cu") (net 6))
 (segment (start 63.7 131.9) (end 71.265425 124.334575) (width 0.25) (layer "F.Cu") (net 6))
 (segment (start 71.265425 124.334575) (end 71.265425 119.769725) (width 0.25) (layer "F.Cu") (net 6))
 (segment (start 120.275 115.5) (end 110.575 105.8) (width 0.25) (layer "B.Cu") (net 3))
 (segment (start 127.84 145.7) (end 127.84 131.9) (width 0.25) (layer "B.Cu") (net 3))
 (segment (start 120.275 119.7) (end 120.275 115.5) (width 0.25) (layer "B.Cu") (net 3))
 (segment (start 120.275 124.335) (end 125.3 129.36) (width 0.25) (layer "B.Cu") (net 3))
 (segment (start 120.275 119.7) (end 120.275 124.335) (width 0.25) (layer "B.Cu") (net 3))
 (segment (start 127.84 131.9) (end 125.3 129.36) (width 0.25) (layer "B.Cu") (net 3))
 (segment (start 125.3 131.9) (end 117.735 124.335) (width 0.25) (layer "B.Cu") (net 4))
 (segment (start 117.735 115.5) (end 108.035 105.8) (width 0.25) (layer "B.Cu") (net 4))
 (segment (start 117.735 124.335) (end 117.735 119.7) (width 0.25) (layer "B.Cu") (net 4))
 (segment (start 117.735 119.7) (end 117.735 115.5) (width 0.25) (layer "B.Cu") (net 4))
 (segment (start 125.3 145.7) (end 125.3 131.9) (width 0.25) (layer "B.Cu") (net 4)))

